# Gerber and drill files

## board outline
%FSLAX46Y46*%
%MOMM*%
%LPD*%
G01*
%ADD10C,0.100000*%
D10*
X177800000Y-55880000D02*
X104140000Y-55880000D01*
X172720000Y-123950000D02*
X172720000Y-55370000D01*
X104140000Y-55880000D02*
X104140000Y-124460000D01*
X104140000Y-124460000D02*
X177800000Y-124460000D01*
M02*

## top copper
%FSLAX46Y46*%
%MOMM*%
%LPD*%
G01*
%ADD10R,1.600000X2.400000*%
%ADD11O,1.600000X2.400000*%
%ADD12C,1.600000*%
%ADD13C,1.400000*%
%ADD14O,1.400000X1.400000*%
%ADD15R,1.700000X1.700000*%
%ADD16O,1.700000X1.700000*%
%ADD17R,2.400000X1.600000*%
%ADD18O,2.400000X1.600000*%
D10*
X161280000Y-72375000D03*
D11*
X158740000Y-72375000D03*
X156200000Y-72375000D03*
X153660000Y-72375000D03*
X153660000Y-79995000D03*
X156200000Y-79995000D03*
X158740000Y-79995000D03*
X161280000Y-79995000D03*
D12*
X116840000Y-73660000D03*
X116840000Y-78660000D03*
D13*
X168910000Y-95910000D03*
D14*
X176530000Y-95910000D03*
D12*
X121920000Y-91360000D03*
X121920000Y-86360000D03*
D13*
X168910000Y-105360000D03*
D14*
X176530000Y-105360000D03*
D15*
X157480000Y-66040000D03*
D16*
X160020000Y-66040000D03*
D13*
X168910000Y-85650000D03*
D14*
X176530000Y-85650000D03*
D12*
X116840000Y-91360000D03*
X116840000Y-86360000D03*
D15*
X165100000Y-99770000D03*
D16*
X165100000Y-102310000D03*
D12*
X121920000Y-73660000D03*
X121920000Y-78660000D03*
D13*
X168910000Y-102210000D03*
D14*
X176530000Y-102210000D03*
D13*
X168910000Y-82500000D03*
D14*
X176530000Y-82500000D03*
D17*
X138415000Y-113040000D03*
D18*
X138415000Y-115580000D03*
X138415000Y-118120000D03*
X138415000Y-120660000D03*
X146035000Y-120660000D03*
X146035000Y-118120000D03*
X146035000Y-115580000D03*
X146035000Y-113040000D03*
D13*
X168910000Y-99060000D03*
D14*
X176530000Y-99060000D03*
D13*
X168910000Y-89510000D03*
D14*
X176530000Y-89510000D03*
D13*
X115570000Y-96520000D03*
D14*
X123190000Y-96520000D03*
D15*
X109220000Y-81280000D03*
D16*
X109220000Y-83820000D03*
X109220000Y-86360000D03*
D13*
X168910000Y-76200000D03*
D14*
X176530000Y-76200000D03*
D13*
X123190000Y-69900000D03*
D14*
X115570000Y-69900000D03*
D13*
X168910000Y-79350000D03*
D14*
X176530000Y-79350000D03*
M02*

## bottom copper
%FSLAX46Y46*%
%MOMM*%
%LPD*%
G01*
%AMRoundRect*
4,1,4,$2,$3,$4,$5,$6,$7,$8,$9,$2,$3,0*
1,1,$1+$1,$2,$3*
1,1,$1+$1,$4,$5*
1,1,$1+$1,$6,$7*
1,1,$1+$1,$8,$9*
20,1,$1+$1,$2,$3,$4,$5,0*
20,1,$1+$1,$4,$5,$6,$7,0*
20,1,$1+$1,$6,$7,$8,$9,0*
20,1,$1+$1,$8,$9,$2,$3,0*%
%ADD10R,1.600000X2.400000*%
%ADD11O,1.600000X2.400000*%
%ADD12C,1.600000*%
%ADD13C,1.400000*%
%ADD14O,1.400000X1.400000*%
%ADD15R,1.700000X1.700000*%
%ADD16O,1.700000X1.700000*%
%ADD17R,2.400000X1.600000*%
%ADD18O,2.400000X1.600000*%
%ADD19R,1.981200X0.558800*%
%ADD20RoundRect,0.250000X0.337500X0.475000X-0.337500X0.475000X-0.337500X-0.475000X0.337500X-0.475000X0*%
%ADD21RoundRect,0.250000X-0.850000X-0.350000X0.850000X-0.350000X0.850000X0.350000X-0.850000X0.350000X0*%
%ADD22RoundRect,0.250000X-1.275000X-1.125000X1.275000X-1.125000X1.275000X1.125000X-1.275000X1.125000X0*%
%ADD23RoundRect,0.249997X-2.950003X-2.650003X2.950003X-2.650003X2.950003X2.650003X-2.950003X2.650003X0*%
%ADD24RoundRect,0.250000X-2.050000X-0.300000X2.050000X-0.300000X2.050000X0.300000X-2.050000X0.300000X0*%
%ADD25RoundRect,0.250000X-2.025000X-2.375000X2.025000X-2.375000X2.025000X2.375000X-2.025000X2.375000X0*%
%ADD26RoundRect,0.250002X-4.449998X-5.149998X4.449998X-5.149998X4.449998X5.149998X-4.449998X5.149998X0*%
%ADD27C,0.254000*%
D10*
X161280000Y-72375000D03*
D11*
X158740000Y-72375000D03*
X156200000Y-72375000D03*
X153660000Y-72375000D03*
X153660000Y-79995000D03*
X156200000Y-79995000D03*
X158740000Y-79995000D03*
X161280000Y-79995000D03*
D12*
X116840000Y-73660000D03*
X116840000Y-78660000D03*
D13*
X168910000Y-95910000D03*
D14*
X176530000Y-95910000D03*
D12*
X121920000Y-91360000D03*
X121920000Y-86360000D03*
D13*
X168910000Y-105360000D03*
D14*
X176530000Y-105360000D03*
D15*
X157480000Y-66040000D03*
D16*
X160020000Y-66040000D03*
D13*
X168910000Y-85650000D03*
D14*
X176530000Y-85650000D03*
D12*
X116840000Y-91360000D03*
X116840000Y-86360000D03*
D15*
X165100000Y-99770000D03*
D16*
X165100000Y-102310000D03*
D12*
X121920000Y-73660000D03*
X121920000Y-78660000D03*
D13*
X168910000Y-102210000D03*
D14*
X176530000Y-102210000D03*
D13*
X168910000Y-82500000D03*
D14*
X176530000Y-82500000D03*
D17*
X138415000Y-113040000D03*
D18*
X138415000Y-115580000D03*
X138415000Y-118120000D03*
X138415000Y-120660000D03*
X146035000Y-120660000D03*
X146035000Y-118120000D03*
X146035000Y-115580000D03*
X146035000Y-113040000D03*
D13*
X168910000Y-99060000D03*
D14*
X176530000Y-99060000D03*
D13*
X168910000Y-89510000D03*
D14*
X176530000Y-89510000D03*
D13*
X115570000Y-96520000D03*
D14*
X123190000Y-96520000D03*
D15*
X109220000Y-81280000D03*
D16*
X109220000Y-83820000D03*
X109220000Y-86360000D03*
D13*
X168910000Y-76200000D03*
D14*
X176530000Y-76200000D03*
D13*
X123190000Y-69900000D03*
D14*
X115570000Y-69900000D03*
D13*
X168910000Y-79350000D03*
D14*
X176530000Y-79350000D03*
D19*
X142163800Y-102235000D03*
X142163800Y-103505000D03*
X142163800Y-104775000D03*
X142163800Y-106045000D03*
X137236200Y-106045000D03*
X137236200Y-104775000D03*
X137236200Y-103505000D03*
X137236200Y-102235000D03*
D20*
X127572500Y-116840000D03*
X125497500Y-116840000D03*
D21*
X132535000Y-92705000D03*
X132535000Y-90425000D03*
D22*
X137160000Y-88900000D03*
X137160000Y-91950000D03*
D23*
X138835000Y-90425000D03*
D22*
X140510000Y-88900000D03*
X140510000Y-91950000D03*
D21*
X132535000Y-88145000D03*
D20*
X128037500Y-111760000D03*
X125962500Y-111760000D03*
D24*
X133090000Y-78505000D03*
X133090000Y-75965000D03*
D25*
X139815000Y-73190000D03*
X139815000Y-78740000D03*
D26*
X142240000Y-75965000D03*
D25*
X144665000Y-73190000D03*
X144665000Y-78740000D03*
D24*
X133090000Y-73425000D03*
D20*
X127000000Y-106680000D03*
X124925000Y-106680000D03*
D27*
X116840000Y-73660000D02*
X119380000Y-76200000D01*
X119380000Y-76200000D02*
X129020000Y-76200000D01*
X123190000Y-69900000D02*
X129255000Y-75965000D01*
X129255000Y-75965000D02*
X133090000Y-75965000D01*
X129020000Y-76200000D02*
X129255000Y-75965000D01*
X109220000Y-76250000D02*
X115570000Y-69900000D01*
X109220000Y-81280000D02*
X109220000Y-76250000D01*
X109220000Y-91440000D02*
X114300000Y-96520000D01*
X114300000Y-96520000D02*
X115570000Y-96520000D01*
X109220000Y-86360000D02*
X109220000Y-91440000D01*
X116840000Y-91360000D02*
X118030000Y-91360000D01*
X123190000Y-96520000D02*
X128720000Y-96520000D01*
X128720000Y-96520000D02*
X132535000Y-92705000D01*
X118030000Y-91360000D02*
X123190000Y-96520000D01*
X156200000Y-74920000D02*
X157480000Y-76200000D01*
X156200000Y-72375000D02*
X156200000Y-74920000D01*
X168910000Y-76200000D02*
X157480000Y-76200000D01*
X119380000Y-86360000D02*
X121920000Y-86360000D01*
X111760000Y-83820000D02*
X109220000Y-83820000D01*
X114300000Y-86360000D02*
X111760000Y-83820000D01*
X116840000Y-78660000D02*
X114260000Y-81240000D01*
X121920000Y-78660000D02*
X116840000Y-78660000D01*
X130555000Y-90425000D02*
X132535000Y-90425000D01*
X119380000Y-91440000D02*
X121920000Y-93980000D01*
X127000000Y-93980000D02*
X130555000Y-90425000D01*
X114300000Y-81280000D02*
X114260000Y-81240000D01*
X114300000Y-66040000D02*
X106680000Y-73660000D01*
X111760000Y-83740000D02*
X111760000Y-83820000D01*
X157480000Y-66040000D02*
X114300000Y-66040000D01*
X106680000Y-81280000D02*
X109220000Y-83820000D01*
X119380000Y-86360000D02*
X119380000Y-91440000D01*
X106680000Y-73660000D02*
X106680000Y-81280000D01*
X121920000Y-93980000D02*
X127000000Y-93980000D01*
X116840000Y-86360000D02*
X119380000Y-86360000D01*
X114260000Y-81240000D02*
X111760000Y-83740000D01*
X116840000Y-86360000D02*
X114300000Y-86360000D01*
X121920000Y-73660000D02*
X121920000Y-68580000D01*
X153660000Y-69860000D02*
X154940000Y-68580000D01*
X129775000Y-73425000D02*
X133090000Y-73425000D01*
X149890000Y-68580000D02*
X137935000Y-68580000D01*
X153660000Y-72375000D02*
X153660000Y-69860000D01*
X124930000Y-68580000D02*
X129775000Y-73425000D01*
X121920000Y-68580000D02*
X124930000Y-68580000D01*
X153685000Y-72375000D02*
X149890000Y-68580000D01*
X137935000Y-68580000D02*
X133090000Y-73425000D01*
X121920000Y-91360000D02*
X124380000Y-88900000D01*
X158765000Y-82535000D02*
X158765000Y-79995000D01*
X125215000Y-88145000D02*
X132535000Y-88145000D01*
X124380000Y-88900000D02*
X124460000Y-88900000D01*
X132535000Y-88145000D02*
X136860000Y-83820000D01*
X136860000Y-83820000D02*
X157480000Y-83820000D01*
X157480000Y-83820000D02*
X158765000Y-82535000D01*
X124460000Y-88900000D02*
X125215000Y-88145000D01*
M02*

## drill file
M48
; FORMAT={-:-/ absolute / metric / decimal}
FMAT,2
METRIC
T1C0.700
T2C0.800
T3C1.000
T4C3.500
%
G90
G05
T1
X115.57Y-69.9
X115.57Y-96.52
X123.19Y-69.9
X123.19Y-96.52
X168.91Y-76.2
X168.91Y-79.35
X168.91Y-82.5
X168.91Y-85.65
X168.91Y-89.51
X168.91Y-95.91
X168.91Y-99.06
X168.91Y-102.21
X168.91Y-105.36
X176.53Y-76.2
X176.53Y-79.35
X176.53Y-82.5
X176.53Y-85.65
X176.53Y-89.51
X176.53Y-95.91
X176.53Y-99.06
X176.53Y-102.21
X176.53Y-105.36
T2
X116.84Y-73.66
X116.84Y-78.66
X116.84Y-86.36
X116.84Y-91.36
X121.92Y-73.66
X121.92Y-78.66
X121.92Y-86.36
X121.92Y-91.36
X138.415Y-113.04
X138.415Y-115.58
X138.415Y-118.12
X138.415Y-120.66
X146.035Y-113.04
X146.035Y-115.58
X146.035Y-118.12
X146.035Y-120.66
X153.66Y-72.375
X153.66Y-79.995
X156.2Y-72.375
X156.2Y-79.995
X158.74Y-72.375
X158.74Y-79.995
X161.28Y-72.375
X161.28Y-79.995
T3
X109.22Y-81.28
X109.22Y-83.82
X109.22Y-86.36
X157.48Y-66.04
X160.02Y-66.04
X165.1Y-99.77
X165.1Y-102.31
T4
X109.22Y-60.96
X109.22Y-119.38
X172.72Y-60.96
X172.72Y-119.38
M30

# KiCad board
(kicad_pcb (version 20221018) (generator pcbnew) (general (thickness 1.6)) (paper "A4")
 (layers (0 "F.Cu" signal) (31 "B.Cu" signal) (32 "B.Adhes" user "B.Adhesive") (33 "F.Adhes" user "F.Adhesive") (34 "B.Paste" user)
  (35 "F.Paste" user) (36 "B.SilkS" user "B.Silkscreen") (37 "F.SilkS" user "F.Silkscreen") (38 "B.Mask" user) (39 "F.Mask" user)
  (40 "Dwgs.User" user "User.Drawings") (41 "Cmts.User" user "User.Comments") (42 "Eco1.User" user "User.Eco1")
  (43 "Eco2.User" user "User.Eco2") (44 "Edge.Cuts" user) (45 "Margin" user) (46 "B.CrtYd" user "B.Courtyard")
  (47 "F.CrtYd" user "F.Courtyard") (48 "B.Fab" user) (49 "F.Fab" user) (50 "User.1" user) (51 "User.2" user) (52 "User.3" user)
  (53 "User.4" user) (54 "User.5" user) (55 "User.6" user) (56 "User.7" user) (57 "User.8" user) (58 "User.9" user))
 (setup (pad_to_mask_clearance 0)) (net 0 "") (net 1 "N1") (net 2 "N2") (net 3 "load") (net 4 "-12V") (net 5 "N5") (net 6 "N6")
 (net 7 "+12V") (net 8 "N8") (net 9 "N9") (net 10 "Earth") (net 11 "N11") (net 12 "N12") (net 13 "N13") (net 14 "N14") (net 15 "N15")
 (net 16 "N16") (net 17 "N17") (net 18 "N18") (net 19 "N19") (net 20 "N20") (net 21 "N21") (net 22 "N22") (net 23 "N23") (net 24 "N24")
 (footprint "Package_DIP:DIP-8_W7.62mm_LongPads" (layer "F.Cu") (at 161.28 72.375 -90)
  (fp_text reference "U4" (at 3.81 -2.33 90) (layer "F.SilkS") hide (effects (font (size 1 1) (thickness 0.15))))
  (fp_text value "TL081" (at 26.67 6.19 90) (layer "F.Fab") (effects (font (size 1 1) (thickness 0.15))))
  (pad "1" thru_hole rect (at 0 0 270) (size 2.4 1.6) (drill 0.8) (layers "*.Cu" "*.Mask") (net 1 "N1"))
  (pad "2" thru_hole oval (at 0 2.54 270) (size 2.4 1.6) (drill 0.8) (layers "*.Cu" "*.Mask") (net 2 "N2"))
  (pad "3" thru_hole oval (at 0 5.08 270) (size 2.4 1.6) (drill 0.8) (layers "*.Cu" "*.Mask") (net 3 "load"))
  (pad "4" thru_hole oval (at 0 7.62 270) (size 2.4 1.6) (drill 0.8) (layers "*.Cu" "*.Mask") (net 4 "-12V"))
  (pad "5" thru_hole oval (at 7.62 7.62 270) (size 2.4 1.6) (drill 0.8) (layers "*.Cu" "*.Mask") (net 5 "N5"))
  (pad "6" thru_hole oval (at 7.62 5.08 270) (size 2.4 1.6) (drill 0.8) (layers "*.Cu" "*.Mask") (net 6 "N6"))
  (pad "7" thru_hole oval (at 7.62 2.54 270) (size 2.4 1.6) (drill 0.8) (layers "*.Cu" "*.Mask") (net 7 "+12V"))
  (pad "8" thru_hole oval (at 7.62 0 270) (size 2.4 1.6) (drill 0.8) (layers "*.Cu" "*.Mask") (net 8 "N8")))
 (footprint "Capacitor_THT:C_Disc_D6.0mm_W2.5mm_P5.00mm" (layer "F.Cu") (at 116.84 73.66 -90)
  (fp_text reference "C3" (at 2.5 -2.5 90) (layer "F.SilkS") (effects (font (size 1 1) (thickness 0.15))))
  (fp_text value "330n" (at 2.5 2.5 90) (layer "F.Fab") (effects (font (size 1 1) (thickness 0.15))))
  (pad "1" thru_hole circle (at 0 0 270) (size 1.6 1.6) (drill 0.8) (layers "*.Cu" "*.Mask") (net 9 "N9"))
  (pad "2" thru_hole circle (at 5 0 270) (size 1.6 1.6) (drill 0.8) (layers "*.Cu" "*.Mask") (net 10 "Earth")))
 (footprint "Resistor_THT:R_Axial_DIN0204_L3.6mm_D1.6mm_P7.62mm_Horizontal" (layer "F.Cu") (at 168.91 95.91)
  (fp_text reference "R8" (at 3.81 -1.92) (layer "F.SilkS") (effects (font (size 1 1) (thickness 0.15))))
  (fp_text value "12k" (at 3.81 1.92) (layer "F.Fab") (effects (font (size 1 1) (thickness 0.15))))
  (pad "1" thru_hole circle (at 0 0) (size 1.4 1.4) (drill 0.7) (layers "*.Cu" "*.Mask") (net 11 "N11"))
  (pad "2" thru_hole oval (at 7.62 0) (size 1.4 1.4) (drill 0.7) (layers "*.Cu" "*.Mask") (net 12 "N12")))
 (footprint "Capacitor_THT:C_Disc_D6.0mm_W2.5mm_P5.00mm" (layer "F.Cu") (at 121.92 91.36 90)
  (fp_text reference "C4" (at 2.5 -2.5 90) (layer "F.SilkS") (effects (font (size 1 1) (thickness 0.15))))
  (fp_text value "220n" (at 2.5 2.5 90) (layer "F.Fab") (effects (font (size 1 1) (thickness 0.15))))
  (pad "1" thru_hole circle (at 0 0 90) (size 1.6 1.6) (drill 0.8) (layers "*.Cu" "*.Mask") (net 7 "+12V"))
  (pad "2" thru_hole circle (at 5 0 90) (size 1.6 1.6) (drill 0.8) (layers "*.Cu" "*.Mask") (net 10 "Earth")))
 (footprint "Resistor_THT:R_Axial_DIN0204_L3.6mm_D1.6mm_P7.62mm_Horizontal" (layer "F.Cu") (at 168.91 105.36)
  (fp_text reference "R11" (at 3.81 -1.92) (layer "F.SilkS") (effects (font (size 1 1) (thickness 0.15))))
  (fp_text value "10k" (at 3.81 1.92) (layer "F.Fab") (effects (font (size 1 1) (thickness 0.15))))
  (pad "1" thru_hole circle (at 0 0) (size 1.4 1.4) (drill 0.7) (layers "*.Cu" "*.Mask") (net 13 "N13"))
  (pad "2" thru_hole oval (at 7.62 0) (size 1.4 1.4) (drill 0.7) (layers "*.Cu" "*.Mask") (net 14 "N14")))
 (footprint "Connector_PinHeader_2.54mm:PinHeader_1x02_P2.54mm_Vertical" (layer "F.Cu") (at 157.48 66.04 90)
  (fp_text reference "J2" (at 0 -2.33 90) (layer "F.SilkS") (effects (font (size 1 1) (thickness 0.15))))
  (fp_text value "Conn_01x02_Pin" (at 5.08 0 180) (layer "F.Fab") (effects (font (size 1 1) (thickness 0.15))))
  (pad "1" thru_hole rect (at 0 0 90) (size 1.7 1.7) (drill 1) (layers "*.Cu" "*.Mask") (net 10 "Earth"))
  (pad "2" thru_hole oval (at 0 2.54 90) (size 1.7 1.7) (drill 1) (layers "*.Cu" "*.Mask") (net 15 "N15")))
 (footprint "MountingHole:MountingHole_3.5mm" (layer "F.Cu") (at 172.72 60.96)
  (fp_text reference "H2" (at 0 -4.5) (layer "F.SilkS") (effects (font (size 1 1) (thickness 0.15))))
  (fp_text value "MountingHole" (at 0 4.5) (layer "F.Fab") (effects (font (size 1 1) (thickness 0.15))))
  (pad "" np_thru_hole circle (at 0 0) (size 3.5 3.5) (drill 3.5) (layers "*.Cu" "*.Mask")))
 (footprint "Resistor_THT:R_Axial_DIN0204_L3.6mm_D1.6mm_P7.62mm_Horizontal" (layer "F.Cu") (at 168.91 85.65)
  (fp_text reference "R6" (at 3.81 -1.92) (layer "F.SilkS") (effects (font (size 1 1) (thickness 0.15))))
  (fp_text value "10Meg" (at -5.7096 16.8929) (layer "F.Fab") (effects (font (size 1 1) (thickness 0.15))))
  (pad "1" thru_hole circle (at 0 0) (size 1.4 1.4) (drill 0.7) (layers "*.Cu" "*.Mask") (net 3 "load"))
  (pad "2" thru_hole oval (at 7.62 0) (size 1.4 1.4) (drill 0.7) (layers "*.Cu" "*.Mask") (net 15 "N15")))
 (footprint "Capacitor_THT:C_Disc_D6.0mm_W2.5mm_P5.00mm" (layer "F.Cu") (at 116.84 91.36 90)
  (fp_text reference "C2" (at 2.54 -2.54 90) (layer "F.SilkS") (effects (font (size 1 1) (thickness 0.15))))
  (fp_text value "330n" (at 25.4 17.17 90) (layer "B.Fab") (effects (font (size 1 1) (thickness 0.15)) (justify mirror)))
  (pad "1" thru_hole circle (at 0 0 90) (size 1.6 1.6) (drill 0.8) (layers "*.Cu" "*.Mask") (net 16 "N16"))
  (pad "2" thru_hole circle (at 5 0 90) (size 1.6 1.6) (drill 0.8) (layers "*.Cu" "*.Mask") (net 10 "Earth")))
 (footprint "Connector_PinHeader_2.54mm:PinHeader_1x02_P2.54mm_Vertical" (layer "F.Cu") (at 165.1 99.77)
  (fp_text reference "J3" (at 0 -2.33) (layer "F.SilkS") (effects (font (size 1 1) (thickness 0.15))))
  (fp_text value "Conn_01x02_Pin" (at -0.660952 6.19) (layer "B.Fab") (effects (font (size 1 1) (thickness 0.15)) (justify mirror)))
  (pad "1" thru_hole rect (at 0 0) (size 1.7 1.7) (drill 1) (layers "*.Cu" "*.Mask") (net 13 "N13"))
  (pad "2" thru_hole oval (at 0 2.54) (size 1.7 1.7) (drill 1) (layers "*.Cu" "*.Mask") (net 10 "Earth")))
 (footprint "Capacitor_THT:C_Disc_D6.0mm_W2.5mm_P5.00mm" (layer "F.Cu") (at 121.92 73.66 -90)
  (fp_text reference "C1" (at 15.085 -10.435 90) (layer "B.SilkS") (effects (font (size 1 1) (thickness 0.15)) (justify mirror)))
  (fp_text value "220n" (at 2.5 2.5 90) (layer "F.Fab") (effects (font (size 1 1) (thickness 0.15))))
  (pad "1" thru_hole circle (at 0 0 270) (size 1.6 1.6) (drill 0.8) (layers "*.Cu" "*.Mask") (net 4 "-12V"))
  (pad "2" thru_hole circle (at 5 0 270) (size 1.6 1.6) (drill 0.8) (layers "*.Cu" "*.Mask") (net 10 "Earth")))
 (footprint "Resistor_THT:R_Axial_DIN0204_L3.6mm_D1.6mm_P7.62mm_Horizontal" (layer "F.Cu") (at 168.91 102.21)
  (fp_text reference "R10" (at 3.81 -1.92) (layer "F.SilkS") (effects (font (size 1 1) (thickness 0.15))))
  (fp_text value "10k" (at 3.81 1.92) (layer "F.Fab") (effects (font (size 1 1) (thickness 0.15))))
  (pad "1" thru_hole circle (at 0 0) (size 1.4 1.4) (drill 0.7) (layers "*.Cu" "*.Mask") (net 14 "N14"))
  (pad "2" thru_hole oval (at 7.62 0) (size 1.4 1.4) (drill 0.7) (layers "*.Cu" "*.Mask") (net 11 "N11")))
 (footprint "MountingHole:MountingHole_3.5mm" (layer "F.Cu") (at 109.22 119.38)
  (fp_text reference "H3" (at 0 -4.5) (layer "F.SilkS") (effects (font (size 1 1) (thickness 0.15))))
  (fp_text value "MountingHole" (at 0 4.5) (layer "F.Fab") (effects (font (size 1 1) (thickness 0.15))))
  (pad "" np_thru_hole circle (at 0 0) (size 3.5 3.5) (drill 3.5) (layers "*.Cu" "*.Mask")))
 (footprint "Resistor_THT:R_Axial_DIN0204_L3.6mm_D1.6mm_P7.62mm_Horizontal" (layer "F.Cu") (at 168.91 82.5)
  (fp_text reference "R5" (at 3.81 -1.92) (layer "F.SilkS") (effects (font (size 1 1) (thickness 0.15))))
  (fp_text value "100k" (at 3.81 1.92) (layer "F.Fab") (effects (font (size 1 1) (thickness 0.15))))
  (pad "1" thru_hole circle (at 0 0) (size 1.4 1.4) (drill 0.7) (layers "*.Cu" "*.Mask") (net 10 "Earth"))
  (pad "2" thru_hole oval (at 7.62 0) (size 1.4 1.4) (drill 0.7) (layers "*.Cu" "*.Mask") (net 2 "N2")))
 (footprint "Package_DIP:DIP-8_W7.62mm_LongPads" (layer "F.Cu") (at 138.415 113.04)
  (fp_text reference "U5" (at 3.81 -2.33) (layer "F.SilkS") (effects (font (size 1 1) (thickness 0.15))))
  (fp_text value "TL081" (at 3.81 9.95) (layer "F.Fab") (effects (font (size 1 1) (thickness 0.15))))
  (pad "1" thru_hole rect (at 0 0) (size 2.4 1.6) (drill 0.8) (layers "*.Cu" "*.Mask") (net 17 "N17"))
  (pad "2" thru_hole oval (at 0 2.54) (size 2.4 1.6) (drill 0.8) (layers "*.Cu" "*.Mask") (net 10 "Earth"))
  (pad "3" thru_hole oval (at 0 5.08) (size 2.4 1.6) (drill 0.8) (layers "*.Cu" "*.Mask") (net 14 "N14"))
  (pad "4" thru_hole oval (at 0 7.62) (size 2.4 1.6) (drill 0.8) (layers "*.Cu" "*.Mask") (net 4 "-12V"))
  (pad "5" thru_hole oval (at 7.62 7.62) (size 2.4 1.6) (drill 0.8) (layers "*.Cu" "*.Mask") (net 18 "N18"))
  (pad "6" thru_hole oval (at 7.62 5.08) (size 2.4 1.6) (drill 0.8) (layers "*.Cu" "*.Mask") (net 13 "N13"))
  (pad "7" thru_hole oval (at 7.62 2.54) (size 2.4 1.6) (drill 0.8) (layers "*.Cu" "*.Mask") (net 7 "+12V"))
  (pad "8" thru_hole oval (at 7.62 0) (size 2.4 1.6) (drill 0.8) (layers "*.Cu" "*.Mask") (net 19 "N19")))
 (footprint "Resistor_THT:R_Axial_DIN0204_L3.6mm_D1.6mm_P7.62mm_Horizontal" (layer "F.Cu") (at 168.91 99.06)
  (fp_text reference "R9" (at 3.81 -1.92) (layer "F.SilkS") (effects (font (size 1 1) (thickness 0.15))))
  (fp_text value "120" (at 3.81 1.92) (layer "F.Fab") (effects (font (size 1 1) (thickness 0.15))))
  (pad "1" thru_hole circle (at 0 0) (size 1.4 1.4) (drill 0.7) (layers "*.Cu" "*.Mask") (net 12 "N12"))
  (pad "2" thru_hole oval (at 7.62 0) (size 1.4 1.4) (drill 0.7) (layers "*.Cu" "*.Mask") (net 10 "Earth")))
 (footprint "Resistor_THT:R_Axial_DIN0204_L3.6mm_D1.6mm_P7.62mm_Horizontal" (layer "F.Cu") (at 168.91 89.51)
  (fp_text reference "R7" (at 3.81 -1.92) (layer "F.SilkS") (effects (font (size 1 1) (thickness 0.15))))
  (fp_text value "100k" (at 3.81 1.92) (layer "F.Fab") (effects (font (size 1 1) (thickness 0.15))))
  (pad "1" thru_hole circle (at 0 0) (size 1.4 1.4) (drill 0.7) (layers "*.Cu" "*.Mask") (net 12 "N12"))
  (pad "2" thru_hole oval (at 7.62 0) (size 1.4 1.4) (drill 0.7) (layers "*.Cu" "*.Mask") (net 3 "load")))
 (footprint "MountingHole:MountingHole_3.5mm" (layer "F.Cu") (at 109.22 60.96)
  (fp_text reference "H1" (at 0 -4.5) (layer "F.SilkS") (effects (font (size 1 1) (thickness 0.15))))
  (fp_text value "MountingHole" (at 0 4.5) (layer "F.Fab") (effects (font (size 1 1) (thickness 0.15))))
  (pad "" np_thru_hole circle (at 0 0) (size 3.5 3.5) (drill 3.5) (layers "*.Cu" "*.Mask")))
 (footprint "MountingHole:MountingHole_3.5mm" (layer "F.Cu") (at 172.72 119.38)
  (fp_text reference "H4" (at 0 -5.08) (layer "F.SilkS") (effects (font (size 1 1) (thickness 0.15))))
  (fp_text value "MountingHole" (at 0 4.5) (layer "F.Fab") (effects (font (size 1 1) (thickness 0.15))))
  (pad "" np_thru_hole circle (at 0 0) (size 3.5 3.5) (drill 3.5) (layers "*.Cu" "*.Mask")))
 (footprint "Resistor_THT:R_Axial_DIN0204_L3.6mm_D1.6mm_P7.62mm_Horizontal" (layer "F.Cu") (at 115.57 96.52)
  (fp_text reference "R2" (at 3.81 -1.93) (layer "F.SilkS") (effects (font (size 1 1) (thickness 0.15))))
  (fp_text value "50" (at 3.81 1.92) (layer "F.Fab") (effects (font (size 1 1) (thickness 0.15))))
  (pad "1" thru_hole circle (at 0 0) (size 1.4 1.4) (drill 0.7) (layers "*.Cu" "*.Mask") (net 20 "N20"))
  (pad "2" thru_hole oval (at 7.62 0) (size 1.4 1.4) (drill 0.7) (layers "*.Cu" "*.Mask") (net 16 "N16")))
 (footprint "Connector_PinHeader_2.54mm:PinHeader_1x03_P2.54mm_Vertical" (layer "F.Cu") (at 109.22 81.28)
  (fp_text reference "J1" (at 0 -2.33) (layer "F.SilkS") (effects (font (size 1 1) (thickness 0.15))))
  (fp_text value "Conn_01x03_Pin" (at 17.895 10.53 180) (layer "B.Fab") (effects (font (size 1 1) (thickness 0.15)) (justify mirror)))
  (pad "1" thru_hole rect (at 0 0) (size 1.7 1.7) (drill 1) (layers "*.Cu" "*.Mask") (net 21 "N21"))
  (pad "2" thru_hole oval (at 0 2.54) (size 1.7 1.7) (drill 1) (layers "*.Cu" "*.Mask") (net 10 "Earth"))
  (pad "3" thru_hole oval (at 0 5.08) (size 1.7 1.7) (drill 1) (layers "*.Cu" "*.Mask") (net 20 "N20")))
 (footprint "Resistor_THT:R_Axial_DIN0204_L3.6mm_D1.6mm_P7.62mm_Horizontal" (layer "F.Cu") (at 168.91 76.2)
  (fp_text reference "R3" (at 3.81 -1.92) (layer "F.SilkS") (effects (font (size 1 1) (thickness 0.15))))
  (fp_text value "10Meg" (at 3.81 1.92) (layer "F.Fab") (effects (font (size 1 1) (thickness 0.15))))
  (pad "1" thru_hole circle (at 0 0) (size 1.4 1.4) (drill 0.7) (layers "*.Cu" "*.Mask") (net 3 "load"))
  (pad "2" thru_hole oval (at 7.62 0) (size 1.4 1.4) (drill 0.7) (layers "*.Cu" "*.Mask") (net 6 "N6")))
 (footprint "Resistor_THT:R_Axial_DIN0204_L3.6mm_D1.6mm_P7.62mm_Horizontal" (layer "F.Cu") (at 123.19 69.9 180)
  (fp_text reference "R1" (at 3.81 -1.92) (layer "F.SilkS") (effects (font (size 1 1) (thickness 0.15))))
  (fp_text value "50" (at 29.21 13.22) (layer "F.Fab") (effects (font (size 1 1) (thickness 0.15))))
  (pad "1" thru_hole circle (at 0 0 180) (size 1.4 1.4) (drill 0.7) (layers "*.Cu" "*.Mask") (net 9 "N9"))
  (pad "2" thru_hole oval (at 7.62 0 180) (size 1.4 1.4) (drill 0.7) (layers "*.Cu" "*.Mask") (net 21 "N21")))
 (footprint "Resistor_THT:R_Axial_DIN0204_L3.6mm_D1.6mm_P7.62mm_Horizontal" (layer "F.Cu") (at 168.91 79.35)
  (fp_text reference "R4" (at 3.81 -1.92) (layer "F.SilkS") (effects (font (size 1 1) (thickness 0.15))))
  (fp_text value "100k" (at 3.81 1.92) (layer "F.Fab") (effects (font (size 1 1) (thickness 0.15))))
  (pad "1" thru_hole circle (at 0 0) (size 1.4 1.4) (drill 0.7) (layers "*.Cu" "*.Mask") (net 2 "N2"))
  (pad "2" thru_hole oval (at 7.62 0) (size 1.4 1.4) (drill 0.7) (layers "*.Cu" "*.Mask") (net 6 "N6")))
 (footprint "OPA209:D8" (layer "B.Cu") (at 139.7 104.14 180)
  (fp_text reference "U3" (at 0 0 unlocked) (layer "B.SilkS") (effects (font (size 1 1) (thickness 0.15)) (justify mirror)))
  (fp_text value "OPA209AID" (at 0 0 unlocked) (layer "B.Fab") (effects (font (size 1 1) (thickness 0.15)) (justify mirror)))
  (pad "1" smd rect (at -2.4638 1.905 180) (size 1.9812 0.5588) (layers "B.Cu" "B.Paste" "B.Mask") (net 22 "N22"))
  (pad "2" smd rect (at -2.4638 0.635 180) (size 1.9812 0.5588) (layers "B.Cu" "B.Paste" "B.Mask") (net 3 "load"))
  (pad "3" smd rect (at -2.4638 -0.635 180) (size 1.9812 0.5588) (layers "B.Cu" "B.Paste" "B.Mask") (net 10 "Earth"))
  (pad "4" smd rect (at -2.4638 -1.905 180) (size 1.9812 0.5588) (layers "B.Cu" "B.Paste" "B.Mask") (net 4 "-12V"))
  (pad "5" smd rect (at 2.4638 -1.905 180) (size 1.9812 0.5588) (layers "B.Cu" "B.Paste" "B.Mask") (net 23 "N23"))
  (pad "6" smd rect (at 2.4638 -0.635 180) (size 1.9812 0.5588) (layers "B.Cu" "B.Paste" "B.Mask") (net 11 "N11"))
  (pad "7" smd rect (at 2.4638 0.635 180) (size 1.9812 0.5588) (layers "B.Cu" "B.Paste" "B.Mask") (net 7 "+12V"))
  (pad "8" smd rect (at 2.4638 1.905 180) (size 1.9812 0.5588) (layers "B.Cu" "B.Paste" "B.Mask") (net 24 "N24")))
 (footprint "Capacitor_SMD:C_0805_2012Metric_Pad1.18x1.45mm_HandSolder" (layer "B.Cu") (at 126.535 116.84 180)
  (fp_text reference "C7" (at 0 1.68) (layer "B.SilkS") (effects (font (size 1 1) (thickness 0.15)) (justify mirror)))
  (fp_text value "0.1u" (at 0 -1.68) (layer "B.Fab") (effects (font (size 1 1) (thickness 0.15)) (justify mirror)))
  (pad "1" smd roundrect (at -1.0375 0 180) (size 1.175 1.45) (layers "B.Cu" "B.Paste" "B.Mask") (roundrect_rratio 0.2127659574)
   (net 4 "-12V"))
  (pad "2" smd roundrect (at 1.0375 0 180) (size 1.175 1.45) (layers "B.Cu" "B.Paste" "B.Mask") (roundrect_rratio 0.2127659574)
   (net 10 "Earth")))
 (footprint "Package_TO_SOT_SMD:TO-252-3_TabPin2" (layer "B.Cu") (at 137.575 90.425)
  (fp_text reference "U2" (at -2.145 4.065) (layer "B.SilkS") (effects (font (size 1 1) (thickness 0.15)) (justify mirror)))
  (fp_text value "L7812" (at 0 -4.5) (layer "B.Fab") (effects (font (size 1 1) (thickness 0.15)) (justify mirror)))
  (pad "1" smd roundrect (at -5.04 2.28) (size 2.2 1.2) (layers "B.Cu" "B.Paste" "B.Mask") (roundrect_rratio 0.2083333333) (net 16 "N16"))
  (pad "2" smd roundrect (at -5.04 0) (size 2.2 1.2) (layers "B.Cu" "B.Paste" "B.Mask") (roundrect_rratio 0.2083333333) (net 10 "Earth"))
  (pad "2" smd roundrect (at -0.415 -1.525) (size 3.05 2.75) (layers "B.Cu" "B.Paste") (roundrect_rratio 0.09090909091) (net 10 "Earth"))
  (pad "2" smd roundrect (at -0.415 1.525) (size 3.05 2.75) (layers "B.Cu" "B.Paste") (roundrect_rratio 0.09090909091) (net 10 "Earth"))
  (pad "2" smd roundrect (at 1.26 0) (size 6.4 5.8) (layers "B.Cu" "B.Mask") (roundrect_rratio 0.04310293103) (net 10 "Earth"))
  (pad "2" smd roundrect (at 2.935 -1.525) (size 3.05 2.75) (layers "B.Cu" "B.Paste") (roundrect_rratio 0.09090909091) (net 10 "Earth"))
  (pad "2" smd roundrect (at 2.935 1.525) (size 3.05 2.75) (layers "B.Cu" "B.Paste") (roundrect_rratio 0.09090909091) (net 10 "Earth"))
  (pad "3" smd roundrect (at -5.04 -2.28) (size 2.2 1.2) (layers "B.Cu" "B.Paste" "B.Mask") (roundrect_rratio 0.2083333333) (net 7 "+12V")))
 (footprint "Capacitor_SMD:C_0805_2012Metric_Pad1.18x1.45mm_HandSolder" (layer "B.Cu") (at 127 111.76 180)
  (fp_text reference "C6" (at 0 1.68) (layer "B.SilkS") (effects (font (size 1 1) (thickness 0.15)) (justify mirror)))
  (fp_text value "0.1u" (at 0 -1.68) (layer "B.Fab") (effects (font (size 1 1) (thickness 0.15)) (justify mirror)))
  (pad "1" smd roundrect (at -1.0375 0 180) (size 1.175 1.45) (layers "B.Cu" "B.Paste" "B.Mask") (roundrect_rratio 0.2127659574)
   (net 7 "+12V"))
  (pad "2" smd roundrect (at 1.0375 0 180) (size 1.175 1.45) (layers "B.Cu" "B.Paste" "B.Mask") (roundrect_rratio 0.2127659574)
   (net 10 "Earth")))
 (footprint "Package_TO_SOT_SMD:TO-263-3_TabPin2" (layer "B.Cu") (at 140.74 75.965)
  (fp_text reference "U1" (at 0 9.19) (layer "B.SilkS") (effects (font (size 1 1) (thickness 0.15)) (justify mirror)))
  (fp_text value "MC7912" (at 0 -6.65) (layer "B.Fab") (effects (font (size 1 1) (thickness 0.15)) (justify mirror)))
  (pad "1" smd roundrect (at -7.65 2.54) (size 4.6 1.1) (layers "B.Cu" "B.Paste" "B.Mask") (roundrect_rratio 0.2272727273) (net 10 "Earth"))
  (pad "2" smd roundrect (at -7.65 0) (size 4.6 1.1) (layers "B.Cu" "B.Paste" "B.Mask") (roundrect_rratio 0.2272727273) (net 9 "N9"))
  (pad "2" smd roundrect (at -0.925 -2.775) (size 4.55 5.25) (layers "B.Cu" "B.Paste") (roundrect_rratio 0.05494505495) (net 9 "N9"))
  (pad "2" smd roundrect (at -0.925 2.775) (size 4.55 5.25) (layers "B.Cu" "B.Paste") (roundrect_rratio 0.05494505495) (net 9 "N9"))
  (pad "2" smd roundrect (at 1.5 0) (size 9.4 10.8) (layers "B.Cu" "B.Mask") (roundrect_rratio 0.02659595745) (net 9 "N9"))
  (pad "2" smd roundrect (at 3.925 -2.775) (size 4.55 5.25) (layers "B.Cu" "B.Paste") (roundrect_rratio 0.05494505495) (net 9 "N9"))
  (pad "2" smd roundrect (at 3.925 2.775) (size 4.55 5.25) (layers "B.Cu" "B.Paste") (roundrect_rratio 0.05494505495) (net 9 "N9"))
  (pad "3" smd roundrect (at -7.65 -2.54) (size 4.6 1.1) (layers "B.Cu" "B.Paste" "B.Mask") (roundrect_rratio 0.2272727273) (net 4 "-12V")))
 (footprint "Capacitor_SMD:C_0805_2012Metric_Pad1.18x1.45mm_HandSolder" (layer "B.Cu") (at 125.9625 106.68 180)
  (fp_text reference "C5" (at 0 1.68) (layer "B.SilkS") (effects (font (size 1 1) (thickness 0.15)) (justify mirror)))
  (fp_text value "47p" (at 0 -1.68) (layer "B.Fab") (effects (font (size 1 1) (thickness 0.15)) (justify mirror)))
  (pad "1" smd roundrect (at -1.0375 0 180) (size 1.175 1.45) (layers "B.Cu" "B.Paste" "B.Mask") (roundrect_rratio 0.2127659574)
   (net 3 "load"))
  (pad "2" smd roundrect (at 1.0375 0 180) (size 1.175 1.45) (layers "B.Cu" "B.Paste" "B.Mask") (roundrect_rratio 0.2127659574)
   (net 10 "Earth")))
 (gr_line (start 177.8 55.88) (end 104.14 55.88) (stroke (width 0.1) (type default)) (layer "Edge.Cuts"))
 (gr_line (start 172.72 123.95) (end 172.72 55.37) (stroke (width 0.1) (type default)) (layer "Edge.Cuts"))
 (gr_line (start 104.14 55.88) (end 104.14 124.46) (stroke (width 0.1) (type default)) (layer "Edge.Cuts"))
 (gr_line (start 104.14 124.46) (end 177.8 124.46) (stroke (width 0.1) (type default)) (layer "Edge.Cuts"))
 (segment (start 116.84 73.66) (end 119.38 76.2) (width 0.254) (layer "B.Cu") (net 9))
 (segment (start 119.38 76.2) (end 129.02 76.2) (width 0.254) (layer "B.Cu") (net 9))
 (segment (start 123.19 69.9) (end 129.255 75.965) (width 0.254) (layer "B.Cu") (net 9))
 (segment (start 129.255 75.965) (end 133.09 75.965) (width 0.254) (layer "B.Cu") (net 9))
 (segment (start 129.02 76.2) (end 129.255 75.965) (width 0.254) (layer "B.Cu") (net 9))
 (segment (start 109.22 76.25) (end 115.57 69.9) (width 0.254) (layer "B.Cu") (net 21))
 (segment (start 109.22 81.28) (end 109.22 76.25) (width 0.254) (layer "B.Cu") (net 21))
 (segment (start 109.22 91.44) (end 114.3 96.52) (width 0.254) (layer "B.Cu") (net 20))
 (segment (start 114.3 96.52) (end 115.57 96.52) (width 0.254) (layer "B.Cu") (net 20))
 (segment (start 109.22 86.36) (end 109.22 91.44) (width 0.254) (layer "B.Cu") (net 20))
 (segment (start 116.84 91.36) (end 118.03 91.36) (width 0.254) (layer "B.Cu") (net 16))
 (segment (start 123.19 96.52) (end 128.72 96.52) (width 0.254) (layer "B.Cu") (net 16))
 (segment (start 128.72 96.52) (end 132.535 92.705) (width 0.254) (layer "B.Cu") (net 16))
 (segment (start 118.03 91.36) (end 123.19 96.52) (width 0.254) (layer "B.Cu") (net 16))
 (segment (start 156.2 74.92) (end 157.48 76.2) (width 0.254) (layer "B.Cu") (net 3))
 (segment (start 156.2 72.375) (end 156.2 74.92) (width 0.254) (layer "B.Cu") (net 3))
 (segment (start 168.91 76.2) (end 157.48 76.2) (width 0.254) (layer "B.Cu") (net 3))
 (segment (start 119.38 86.36) (end 121.92 86.36) (width 0.254) (layer "B.Cu") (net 10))
 (segment (start 111.76 83.82) (end 109.22 83.82) (width 0.254) (layer "B.Cu") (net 10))
 (segment (start 114.3 86.36) (end 111.76 83.82) (width 0.254) (layer "B.Cu") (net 10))
 (segment (start 116.84 78.66) (end 114.26 81.24) (width 0.254) (layer "B.Cu") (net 10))
 (segment (start 121.92 78.66) (end 116.84 78.66) (width 0.254) (layer "B.Cu") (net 10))
 (segment (start 130.555 90.425) (end 132.535 90.425) (width 0.254) (layer "B.Cu") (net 10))
 (segment (start 119.38 91.44) (end 121.92 93.98) (width 0.254) (layer "B.Cu") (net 10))
 (segment (start 127 93.98) (end 130.555 90.425) (width 0.254) (layer "B.Cu") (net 10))
 (segment (start 114.3 81.28) (end 114.26 81.24) (width 0.254) (layer "B.Cu") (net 10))
 (segment (start 114.3 66.04) (end 106.68 73.66) (width 0.254) (layer "B.Cu") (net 10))
 (segment (start 111.76 83.74) (end 111.76 83.82) (width 0.254) (layer "B.Cu") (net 10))
 (segment (start 157.48 66.04) (end 114.3 66.04) (width 0.254) (layer "B.Cu") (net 10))
 (segment (start 106.68 81.28) (end 109.22 83.82) (width 0.254) (layer "B.Cu") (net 10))
 (segment (start 119.38 86.36) (end 119.38 91.44) (width 0.254) (layer "B.Cu") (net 10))
 (segment (start 106.68 73.66) (end 106.68 81.28) (width 0.254) (layer "B.Cu") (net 10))
 (segment (start 121.92 93.98) (end 127 93.98) (width 0.254) (layer "B.Cu") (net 10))
 (segment (start 116.84 86.36) (end 119.38 86.36) (width 0.254) (layer "B.Cu") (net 10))
 (segment (start 114.26 81.24) (end 111.76 83.74) (width 0.254) (layer "B.Cu") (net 10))
 (segment (start 116.84 86.36) (end 114.3 86.36) (width 0.254) (layer "B.Cu") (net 10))
 (segment (start 121.92 73.66) (end 121.92 68.58) (width 0.254) (layer "B.Cu") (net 4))
 (segment (start 153.66 69.86) (end 154.94 68.58) (width 0.254) (layer "B.Cu") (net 4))
 (segment (start 129.775 73.425) (end 133.09 73.425) (width 0.254) (layer "B.Cu") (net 4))
 (segment (start 149.89 68.58) (end 137.935 68.58) (width 0.254) (layer "B.Cu") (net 4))
 (segment (start 153.66 72.375) (end 153.66 69.86) (width 0.254) (layer "B.Cu") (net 4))
 (segment (start 124.93 68.58) (end 129.775 73.425) (width 0.254) (layer "B.Cu") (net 4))
 (segment (start 121.92 68.58) (end 124.93 68.58) (width 0.254) (layer "B.Cu") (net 4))
 (segment (start 153.685 72.375) (end 149.89 68.58) (width 0.254) (layer "B.Cu") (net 4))
 (segment (start 137.935 68.58) (end 133.09 73.425) (width 0.254) (layer "B.Cu") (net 4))
 (segment (start 121.92 91.36) (end 124.38 88.9) (width 0.254) (layer "B.Cu") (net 7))
 (segment (start 158.765 82.535) (end 158.765 79.995) (width 0.254) (layer "B.Cu") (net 7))
 (segment (start 125.215 88.145) (end 132.535 88.145) (width 0.254) (layer "B.Cu") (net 7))
 (segment (start 124.38 88.9) (end 124.46 88.9) (width 0.254) (layer "B.Cu") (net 7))
 (segment (start 132.535 88.145) (end 136.86 83.82) (width 0.254) (layer "B.Cu") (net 7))
 (segment (start 136.86 83.82) (end 157.48 83.82) (width 0.254) (layer "B.Cu") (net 7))
 (segment (start 157.48 83.82) (end 158.765 82.535) (width 0.254) (layer "B.Cu") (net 7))
 (segment (start 124.46 88.9) (end 125.215 88.145) (width 0.254) (layer "B.Cu") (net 7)))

